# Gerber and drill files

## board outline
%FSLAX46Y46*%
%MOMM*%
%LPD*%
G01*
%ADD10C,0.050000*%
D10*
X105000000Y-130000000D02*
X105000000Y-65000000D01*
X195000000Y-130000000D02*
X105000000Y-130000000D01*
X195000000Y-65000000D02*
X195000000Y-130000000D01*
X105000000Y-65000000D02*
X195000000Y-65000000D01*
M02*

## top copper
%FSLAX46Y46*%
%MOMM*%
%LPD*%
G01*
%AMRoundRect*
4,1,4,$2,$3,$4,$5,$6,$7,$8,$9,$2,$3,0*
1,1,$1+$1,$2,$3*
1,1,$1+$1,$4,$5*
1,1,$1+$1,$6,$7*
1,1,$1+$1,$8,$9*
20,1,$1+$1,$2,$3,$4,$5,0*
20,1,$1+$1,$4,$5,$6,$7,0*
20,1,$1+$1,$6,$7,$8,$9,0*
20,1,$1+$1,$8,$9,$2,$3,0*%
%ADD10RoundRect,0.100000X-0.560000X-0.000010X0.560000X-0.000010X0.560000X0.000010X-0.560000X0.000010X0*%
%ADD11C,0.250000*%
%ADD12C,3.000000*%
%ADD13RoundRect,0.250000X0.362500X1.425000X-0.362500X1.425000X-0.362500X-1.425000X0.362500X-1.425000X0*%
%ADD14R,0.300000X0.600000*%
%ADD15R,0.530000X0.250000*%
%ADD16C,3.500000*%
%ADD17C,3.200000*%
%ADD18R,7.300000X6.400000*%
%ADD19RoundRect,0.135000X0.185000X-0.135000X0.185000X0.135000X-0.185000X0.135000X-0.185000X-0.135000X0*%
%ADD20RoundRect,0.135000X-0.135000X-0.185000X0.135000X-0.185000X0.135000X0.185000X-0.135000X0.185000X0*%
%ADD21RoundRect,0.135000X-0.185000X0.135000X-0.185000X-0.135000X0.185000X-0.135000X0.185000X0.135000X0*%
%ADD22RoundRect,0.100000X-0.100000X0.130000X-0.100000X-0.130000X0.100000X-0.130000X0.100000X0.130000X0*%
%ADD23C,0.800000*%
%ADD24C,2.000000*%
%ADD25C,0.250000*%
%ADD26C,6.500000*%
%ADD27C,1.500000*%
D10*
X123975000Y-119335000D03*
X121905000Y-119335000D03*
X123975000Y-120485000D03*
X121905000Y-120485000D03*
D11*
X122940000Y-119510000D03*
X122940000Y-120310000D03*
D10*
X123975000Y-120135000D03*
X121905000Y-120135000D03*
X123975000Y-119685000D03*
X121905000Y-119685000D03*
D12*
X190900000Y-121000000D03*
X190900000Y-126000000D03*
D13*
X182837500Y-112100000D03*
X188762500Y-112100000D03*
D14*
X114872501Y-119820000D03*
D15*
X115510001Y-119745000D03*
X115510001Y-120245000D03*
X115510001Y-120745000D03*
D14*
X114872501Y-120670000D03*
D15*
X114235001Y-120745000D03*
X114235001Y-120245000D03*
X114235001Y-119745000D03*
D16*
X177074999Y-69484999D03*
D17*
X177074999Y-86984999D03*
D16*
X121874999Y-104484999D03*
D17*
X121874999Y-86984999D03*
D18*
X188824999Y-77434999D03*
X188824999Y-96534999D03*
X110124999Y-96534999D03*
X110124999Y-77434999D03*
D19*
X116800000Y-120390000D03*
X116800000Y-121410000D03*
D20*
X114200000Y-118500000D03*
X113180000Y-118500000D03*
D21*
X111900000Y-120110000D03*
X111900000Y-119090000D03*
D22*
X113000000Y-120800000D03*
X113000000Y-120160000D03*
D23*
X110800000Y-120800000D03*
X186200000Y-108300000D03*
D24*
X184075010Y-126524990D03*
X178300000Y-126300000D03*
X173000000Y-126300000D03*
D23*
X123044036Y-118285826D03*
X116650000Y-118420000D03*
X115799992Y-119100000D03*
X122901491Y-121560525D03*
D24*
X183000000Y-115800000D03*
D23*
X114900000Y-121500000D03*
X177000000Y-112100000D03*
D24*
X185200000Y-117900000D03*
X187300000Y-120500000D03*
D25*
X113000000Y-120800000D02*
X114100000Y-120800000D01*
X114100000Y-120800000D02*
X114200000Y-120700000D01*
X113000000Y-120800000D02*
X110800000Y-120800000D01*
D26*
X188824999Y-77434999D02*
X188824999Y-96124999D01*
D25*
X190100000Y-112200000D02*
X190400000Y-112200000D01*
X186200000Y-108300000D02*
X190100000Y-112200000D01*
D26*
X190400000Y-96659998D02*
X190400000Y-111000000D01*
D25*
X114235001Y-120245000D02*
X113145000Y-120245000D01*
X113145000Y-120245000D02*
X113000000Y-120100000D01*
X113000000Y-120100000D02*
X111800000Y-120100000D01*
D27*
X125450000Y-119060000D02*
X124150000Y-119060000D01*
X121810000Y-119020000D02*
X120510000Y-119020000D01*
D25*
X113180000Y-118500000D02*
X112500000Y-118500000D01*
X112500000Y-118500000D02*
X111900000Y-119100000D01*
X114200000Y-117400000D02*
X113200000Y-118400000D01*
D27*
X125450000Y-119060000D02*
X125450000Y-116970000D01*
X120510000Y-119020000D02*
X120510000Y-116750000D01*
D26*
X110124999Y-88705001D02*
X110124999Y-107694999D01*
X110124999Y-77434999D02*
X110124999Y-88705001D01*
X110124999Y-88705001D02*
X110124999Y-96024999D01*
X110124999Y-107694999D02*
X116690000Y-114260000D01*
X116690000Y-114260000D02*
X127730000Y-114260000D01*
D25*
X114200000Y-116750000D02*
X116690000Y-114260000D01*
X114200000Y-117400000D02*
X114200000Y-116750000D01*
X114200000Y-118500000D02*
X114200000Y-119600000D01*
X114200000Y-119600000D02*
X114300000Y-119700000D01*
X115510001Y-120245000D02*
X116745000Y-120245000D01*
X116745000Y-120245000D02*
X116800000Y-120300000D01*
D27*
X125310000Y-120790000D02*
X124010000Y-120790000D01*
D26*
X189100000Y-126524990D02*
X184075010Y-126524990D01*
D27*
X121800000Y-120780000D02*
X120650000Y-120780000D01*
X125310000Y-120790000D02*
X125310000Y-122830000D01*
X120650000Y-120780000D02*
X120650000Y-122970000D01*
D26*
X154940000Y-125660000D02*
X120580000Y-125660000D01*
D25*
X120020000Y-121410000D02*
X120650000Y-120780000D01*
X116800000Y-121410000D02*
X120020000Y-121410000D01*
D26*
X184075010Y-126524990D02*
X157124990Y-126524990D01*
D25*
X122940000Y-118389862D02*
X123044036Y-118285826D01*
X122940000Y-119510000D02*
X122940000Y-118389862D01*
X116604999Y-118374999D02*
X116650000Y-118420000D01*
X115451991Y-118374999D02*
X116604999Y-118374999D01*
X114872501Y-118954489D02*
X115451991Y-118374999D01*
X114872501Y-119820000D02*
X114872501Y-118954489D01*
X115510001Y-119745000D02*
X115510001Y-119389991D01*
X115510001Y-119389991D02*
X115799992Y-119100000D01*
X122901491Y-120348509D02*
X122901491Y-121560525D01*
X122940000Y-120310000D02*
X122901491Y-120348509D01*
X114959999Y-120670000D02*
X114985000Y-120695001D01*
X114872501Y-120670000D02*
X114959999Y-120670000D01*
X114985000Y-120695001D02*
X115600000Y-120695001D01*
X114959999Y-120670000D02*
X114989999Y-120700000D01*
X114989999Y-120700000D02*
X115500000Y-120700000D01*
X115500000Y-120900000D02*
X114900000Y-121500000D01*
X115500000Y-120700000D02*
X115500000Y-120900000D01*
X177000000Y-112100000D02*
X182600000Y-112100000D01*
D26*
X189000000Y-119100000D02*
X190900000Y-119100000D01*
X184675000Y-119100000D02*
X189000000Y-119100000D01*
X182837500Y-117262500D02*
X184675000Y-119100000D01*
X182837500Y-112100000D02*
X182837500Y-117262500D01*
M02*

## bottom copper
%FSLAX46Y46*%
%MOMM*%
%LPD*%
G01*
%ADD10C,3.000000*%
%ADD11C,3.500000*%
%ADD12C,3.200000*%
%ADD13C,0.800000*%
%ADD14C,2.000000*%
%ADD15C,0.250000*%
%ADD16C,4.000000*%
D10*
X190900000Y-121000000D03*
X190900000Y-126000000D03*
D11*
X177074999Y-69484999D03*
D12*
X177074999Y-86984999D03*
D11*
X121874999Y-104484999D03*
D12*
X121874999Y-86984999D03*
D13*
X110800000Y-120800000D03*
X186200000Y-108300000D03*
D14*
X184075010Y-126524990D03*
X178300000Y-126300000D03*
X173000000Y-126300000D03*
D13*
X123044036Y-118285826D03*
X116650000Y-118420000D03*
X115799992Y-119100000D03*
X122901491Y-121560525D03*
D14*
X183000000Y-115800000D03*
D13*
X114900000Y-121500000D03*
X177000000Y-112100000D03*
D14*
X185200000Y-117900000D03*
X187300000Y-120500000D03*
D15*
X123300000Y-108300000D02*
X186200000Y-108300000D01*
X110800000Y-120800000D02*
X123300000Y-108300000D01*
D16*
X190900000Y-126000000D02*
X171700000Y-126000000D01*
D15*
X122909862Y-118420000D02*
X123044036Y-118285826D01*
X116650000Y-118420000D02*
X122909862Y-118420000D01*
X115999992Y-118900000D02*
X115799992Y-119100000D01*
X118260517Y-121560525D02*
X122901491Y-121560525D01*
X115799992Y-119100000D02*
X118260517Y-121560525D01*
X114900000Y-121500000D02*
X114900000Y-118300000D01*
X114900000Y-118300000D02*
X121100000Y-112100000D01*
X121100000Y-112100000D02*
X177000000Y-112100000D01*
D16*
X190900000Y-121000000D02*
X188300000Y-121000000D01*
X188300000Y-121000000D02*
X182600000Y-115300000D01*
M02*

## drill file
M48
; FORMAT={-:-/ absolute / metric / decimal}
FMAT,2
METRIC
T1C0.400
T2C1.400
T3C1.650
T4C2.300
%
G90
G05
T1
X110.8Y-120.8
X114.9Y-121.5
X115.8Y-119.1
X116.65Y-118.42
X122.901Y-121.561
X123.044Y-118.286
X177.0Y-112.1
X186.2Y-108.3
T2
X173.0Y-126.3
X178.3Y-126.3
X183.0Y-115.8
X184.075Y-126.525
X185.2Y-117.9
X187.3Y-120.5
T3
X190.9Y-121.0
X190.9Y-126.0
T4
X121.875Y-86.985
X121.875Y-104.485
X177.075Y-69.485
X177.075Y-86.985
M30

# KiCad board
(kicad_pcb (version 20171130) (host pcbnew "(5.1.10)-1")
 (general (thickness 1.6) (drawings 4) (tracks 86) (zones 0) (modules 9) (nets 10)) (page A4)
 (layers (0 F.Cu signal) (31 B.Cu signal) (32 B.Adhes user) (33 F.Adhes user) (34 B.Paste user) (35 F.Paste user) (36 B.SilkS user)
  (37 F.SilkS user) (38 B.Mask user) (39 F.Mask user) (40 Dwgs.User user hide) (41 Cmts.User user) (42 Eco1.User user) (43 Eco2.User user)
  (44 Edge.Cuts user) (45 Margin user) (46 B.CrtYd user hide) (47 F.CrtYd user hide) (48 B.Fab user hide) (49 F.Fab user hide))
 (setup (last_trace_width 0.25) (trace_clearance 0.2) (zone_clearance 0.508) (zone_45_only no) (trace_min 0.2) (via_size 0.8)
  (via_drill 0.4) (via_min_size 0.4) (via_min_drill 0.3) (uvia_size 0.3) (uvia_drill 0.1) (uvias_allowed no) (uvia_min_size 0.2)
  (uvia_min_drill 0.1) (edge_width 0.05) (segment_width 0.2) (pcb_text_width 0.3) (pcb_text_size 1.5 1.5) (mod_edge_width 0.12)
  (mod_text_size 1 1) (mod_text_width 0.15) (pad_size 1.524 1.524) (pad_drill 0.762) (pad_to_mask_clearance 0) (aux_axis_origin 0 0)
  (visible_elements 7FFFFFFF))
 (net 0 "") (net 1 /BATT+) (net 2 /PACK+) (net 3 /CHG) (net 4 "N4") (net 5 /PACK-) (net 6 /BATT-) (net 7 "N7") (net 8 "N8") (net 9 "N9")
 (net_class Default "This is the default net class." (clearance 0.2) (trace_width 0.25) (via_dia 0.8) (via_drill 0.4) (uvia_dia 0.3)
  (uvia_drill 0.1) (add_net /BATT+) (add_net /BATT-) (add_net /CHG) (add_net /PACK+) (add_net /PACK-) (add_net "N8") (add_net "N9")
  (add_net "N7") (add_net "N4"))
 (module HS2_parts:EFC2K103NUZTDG (layer F.Cu) (at 122.94 119.91)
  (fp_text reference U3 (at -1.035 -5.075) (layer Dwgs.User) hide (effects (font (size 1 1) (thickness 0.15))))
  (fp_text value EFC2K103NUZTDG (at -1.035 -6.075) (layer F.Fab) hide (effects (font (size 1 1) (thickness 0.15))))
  (pad 1 smd roundrect (at 1.035 -0.575) (size 1.32 0.2) (layers F.Cu F.Paste F.Mask) (roundrect_rratio 0.5) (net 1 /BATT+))
  (pad 1 smd roundrect (at -1.035 -0.575) (size 1.32 0.2) (layers F.Cu F.Paste F.Mask) (roundrect_rratio 0.5) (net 1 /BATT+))
  (pad 2 smd roundrect (at 1.035 0.575) (size 1.32 0.2) (layers F.Cu F.Paste F.Mask) (roundrect_rratio 0.5) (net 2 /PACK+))
  (pad 2 smd roundrect (at -1.035 0.575) (size 1.32 0.2) (layers F.Cu F.Paste F.Mask) (roundrect_rratio 0.5) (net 2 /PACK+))
  (pad 3 smd circle (at 0 -0.4) (size 0.25 0.25) (layers F.Cu F.Paste F.Mask) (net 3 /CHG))
  (pad 4 smd circle (at 0 0.4) (size 0.25 0.25) (layers F.Cu F.Paste F.Mask) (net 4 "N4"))
  (pad 2 smd roundrect (at 1.035 0.225) (size 1.32 0.2) (layers F.Cu F.Paste F.Mask) (roundrect_rratio 0.5) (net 2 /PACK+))
  (pad 2 smd roundrect (at -1.035 0.225) (size 1.32 0.2) (layers F.Cu F.Paste F.Mask) (roundrect_rratio 0.5) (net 2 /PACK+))
  (pad 1 smd roundrect (at 1.035 -0.225) (size 1.32 0.2) (layers F.Cu F.Paste F.Mask) (roundrect_rratio 0.5) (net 1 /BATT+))
  (pad 1 smd roundrect (at -1.035 -0.225) (size 1.32 0.2) (layers F.Cu F.Paste F.Mask) (roundrect_rratio 0.5) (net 1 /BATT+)))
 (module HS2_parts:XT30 (layer F.Cu) (at 190.9 126 180)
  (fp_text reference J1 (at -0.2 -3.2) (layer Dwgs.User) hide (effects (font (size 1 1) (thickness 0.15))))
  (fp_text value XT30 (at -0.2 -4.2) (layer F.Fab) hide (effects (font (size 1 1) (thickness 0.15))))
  (pad 2 thru_hole circle (at 0 5 180) (size 3 3) (drill 1.65) (layers *.Cu *.Mask) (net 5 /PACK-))
  (pad 1 thru_hole circle (at 0 0 180) (size 3 3) (drill 1.65) (layers *.Cu *.Mask) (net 2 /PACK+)))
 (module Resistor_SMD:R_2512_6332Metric (layer F.Cu) (at 185.8 112.1 180)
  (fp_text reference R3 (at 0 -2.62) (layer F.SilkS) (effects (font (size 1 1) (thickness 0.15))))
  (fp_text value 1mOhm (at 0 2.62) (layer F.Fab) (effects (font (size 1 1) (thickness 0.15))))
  (pad 2 smd roundrect (at 2.9625 0 180) (size 1.225 3.35) (layers F.Cu F.Paste F.Mask) (roundrect_rratio 0.2040816326530612) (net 5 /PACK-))
  (pad 1 smd roundrect (at -2.9625 0 180) (size 1.225 3.35) (layers F.Cu F.Paste F.Mask) (roundrect_rratio 0.2040816326530612)
   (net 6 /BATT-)))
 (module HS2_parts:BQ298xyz (layer F.Cu) (at 114.872501 120.245 270)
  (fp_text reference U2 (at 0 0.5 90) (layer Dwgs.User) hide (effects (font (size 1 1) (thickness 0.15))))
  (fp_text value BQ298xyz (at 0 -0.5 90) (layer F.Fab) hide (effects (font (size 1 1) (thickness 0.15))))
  (pad 8 smd rect (at -0.425 0) (size 0.3 0.6) (layers F.Cu F.Paste F.Mask) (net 3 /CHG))
  (pad 7 smd rect (at -0.5 -0.6375 270) (size 0.25 0.53) (layers F.Cu F.Paste F.Mask) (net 4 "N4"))
  (pad 6 smd rect (at 0 -0.6375 270) (size 0.25 0.53) (layers F.Cu F.Paste F.Mask) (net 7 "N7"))
  (pad 5 smd rect (at 0.5 -0.6375 270) (size 0.25 0.53) (layers F.Cu F.Paste F.Mask) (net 5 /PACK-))
  (pad 4 smd rect (at 0.425 0) (size 0.3 0.6) (layers F.Cu F.Paste F.Mask) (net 5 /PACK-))
  (pad 3 smd rect (at 0.5 0.6375 270) (size 0.25 0.53) (layers F.Cu F.Paste F.Mask) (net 6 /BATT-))
  (pad 2 smd rect (at 0 0.6375 270) (size 0.25 0.53) (layers F.Cu F.Paste F.Mask) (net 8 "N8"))
  (pad 1 smd rect (at -0.5 0.6375 270) (size 0.25 0.53) (layers F.Cu F.Paste F.Mask) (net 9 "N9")))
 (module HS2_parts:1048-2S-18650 (layer F.Cu) (at 121.874999 86.984999)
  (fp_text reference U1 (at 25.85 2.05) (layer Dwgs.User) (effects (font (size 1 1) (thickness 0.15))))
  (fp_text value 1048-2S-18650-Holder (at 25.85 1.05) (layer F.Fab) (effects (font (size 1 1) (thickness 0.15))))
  (pad "" np_thru_hole circle (at 55.2 -17.5) (size 3.5 3.5) (drill 2.3) (layers *.Cu *.Mask))
  (pad "" np_thru_hole circle (at 55.2 0) (size 3.2 3.2) (drill 2.3) (layers *.Cu *.Mask))
  (pad "" np_thru_hole circle (at 0 17.5) (size 3.5 3.5) (drill 2.3) (layers *.Cu *.Mask))
  (pad "" np_thru_hole circle (at 0 0) (size 3.2 3.2) (drill 2.3) (layers *.Cu *.Mask))
  (pad 4 smd rect (at 66.95 -9.55) (size 7.3 6.4) (layers F.Cu F.Paste F.Mask) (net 6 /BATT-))
  (pad 3 smd rect (at 66.95 9.55) (size 7.3 6.4) (layers F.Cu F.Paste F.Mask) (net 6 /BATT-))
  (pad 2 smd rect (at -11.75 9.55) (size 7.3 6.4) (layers F.Cu F.Paste F.Mask) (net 1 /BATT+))
  (pad 1 smd rect (at -11.75 -9.55) (size 7.3 6.4) (layers F.Cu F.Paste F.Mask) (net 1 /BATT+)))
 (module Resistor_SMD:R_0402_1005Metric (layer F.Cu) (at 116.8 120.9 90)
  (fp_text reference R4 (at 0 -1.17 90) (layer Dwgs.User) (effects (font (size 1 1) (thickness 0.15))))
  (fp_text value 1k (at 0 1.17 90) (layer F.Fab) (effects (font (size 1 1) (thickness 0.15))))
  (pad 2 smd roundrect (at 0.51 0 90) (size 0.54 0.64) (layers F.Cu F.Paste F.Mask) (roundrect_rratio 0.25) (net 7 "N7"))
  (pad 1 smd roundrect (at -0.51 0 90) (size 0.54 0.64) (layers F.Cu F.Paste F.Mask) (roundrect_rratio 0.25) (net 2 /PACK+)))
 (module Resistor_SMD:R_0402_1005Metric (layer F.Cu) (at 113.69 118.5)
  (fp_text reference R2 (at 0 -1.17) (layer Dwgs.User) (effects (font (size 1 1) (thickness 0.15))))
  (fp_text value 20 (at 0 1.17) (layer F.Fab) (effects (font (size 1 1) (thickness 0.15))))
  (pad 2 smd roundrect (at 0.51 0) (size 0.54 0.64) (layers F.Cu F.Paste F.Mask) (roundrect_rratio 0.25) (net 9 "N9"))
  (pad 1 smd roundrect (at -0.51 0) (size 0.54 0.64) (layers F.Cu F.Paste F.Mask) (roundrect_rratio 0.25) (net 1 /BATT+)))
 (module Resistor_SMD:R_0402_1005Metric (layer F.Cu) (at 111.9 119.6 270)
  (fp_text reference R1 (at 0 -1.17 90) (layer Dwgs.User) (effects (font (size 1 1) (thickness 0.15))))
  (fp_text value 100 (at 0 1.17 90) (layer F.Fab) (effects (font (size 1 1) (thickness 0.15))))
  (pad 2 smd roundrect (at 0.51 0 270) (size 0.54 0.64) (layers F.Cu F.Paste F.Mask) (roundrect_rratio 0.25) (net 8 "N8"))
  (pad 1 smd roundrect (at -0.51 0 270) (size 0.54 0.64) (layers F.Cu F.Paste F.Mask) (roundrect_rratio 0.25) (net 1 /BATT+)))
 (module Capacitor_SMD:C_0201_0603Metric (layer F.Cu) (at 113 120.48 270)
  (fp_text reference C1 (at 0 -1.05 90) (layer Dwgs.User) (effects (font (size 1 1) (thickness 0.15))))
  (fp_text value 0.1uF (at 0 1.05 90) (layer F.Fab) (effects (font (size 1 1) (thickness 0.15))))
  (pad 2 smd roundrect (at 0.32 0 270) (size 0.46 0.4) (layers F.Cu F.Mask) (roundrect_rratio 0.25) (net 6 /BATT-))
  (pad 1 smd roundrect (at -0.32 0 270) (size 0.46 0.4) (layers F.Cu F.Mask) (roundrect_rratio 0.25) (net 8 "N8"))
  (pad "" smd roundrect (at 0.345 0 270) (size 0.318 0.36) (layers F.Paste) (roundrect_rratio 0.25))
  (pad "" smd roundrect (at -0.345 0 270) (size 0.318 0.36) (layers F.Paste) (roundrect_rratio 0.25)))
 (gr_line (start 105 130) (end 105 65) (layer Edge.Cuts) (width 0.05))
 (gr_line (start 195 130) (end 105 130) (layer Edge.Cuts) (width 0.05))
 (gr_line (start 195 65) (end 195 130) (layer Edge.Cuts) (width 0.05))
 (gr_line (start 105 65) (end 195 65) (layer Edge.Cuts) (width 0.05))
 (segment (start 113 120.8) (end 114.1 120.8) (width 0.25) (layer F.Cu) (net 6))
 (segment (start 114.1 120.8) (end 114.2 120.7) (width 0.25) (layer F.Cu) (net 6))
 (via (at 110.8 120.8) (size 0.8) (drill 0.4) (layers F.Cu B.Cu) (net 6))
 (segment (start 113 120.8) (end 110.8 120.8) (width 0.25) (layer F.Cu) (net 6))
 (segment (start 188.824999 77.434999) (end 188.824999 96.124999) (width 6.5) (layer F.Cu) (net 6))
 (via (at 186.2 108.3) (size 0.8) (drill 0.4) (layers F.Cu B.Cu) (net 6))
 (segment (start 123.3 108.3) (end 186.2 108.3) (width 0.25) (layer B.Cu) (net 6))
 (segment (start 110.8 120.8) (end 123.3 108.3) (width 0.25) (layer B.Cu) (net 6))
 (segment (start 190.1 112.2) (end 190.4 112.2) (width 0.25) (layer F.Cu) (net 6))
 (segment (start 186.2 108.3) (end 190.1 112.2) (width 0.25) (layer F.Cu) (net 6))
 (segment (start 190.4 96.659998) (end 190.4 111) (width 6.5) (layer F.Cu) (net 6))
 (segment (start 114.235001 120.245) (end 113.145 120.245) (width 0.25) (layer F.Cu) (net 8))
 (segment (start 113.145 120.245) (end 113 120.1) (width 0.25) (layer F.Cu) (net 8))
 (segment (start 113 120.1) (end 111.8 120.1) (width 0.25) (layer F.Cu) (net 8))
 (segment (start 125.45 119.06) (end 124.15 119.06) (width 1.5) (layer F.Cu) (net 1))
 (segment (start 121.81 119.02) (end 120.51 119.02) (width 1.5) (layer F.Cu) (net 1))
 (segment (start 113.18 118.5) (end 112.5 118.5) (width 0.25) (layer F.Cu) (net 1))
 (segment (start 112.5 118.5) (end 111.9 119.1) (width 0.25) (layer F.Cu) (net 1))
 (segment (start 114.2 117.4) (end 113.2 118.4) (width 0.25) (layer F.Cu) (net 1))
 (segment (start 125.45 119.06) (end 125.45 116.97) (width 1.5) (layer F.Cu) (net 1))
 (segment (start 120.51 119.02) (end 120.51 116.75) (width 1.5) (layer F.Cu) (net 1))
 (segment (start 110.124999 88.705001) (end 110.124999 107.694999) (width 6.5) (layer F.Cu) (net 1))
 (segment (start 110.124999 77.434999) (end 110.124999 88.705001) (width 6.5) (layer F.Cu) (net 1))
 (segment (start 110.124999 88.705001) (end 110.124999 96.024999) (width 6.5) (layer F.Cu) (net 1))
 (segment (start 110.124999 107.694999) (end 116.69 114.26) (width 6.5) (layer F.Cu) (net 1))
 (segment (start 116.69 114.26) (end 127.73 114.26) (width 6.5) (layer F.Cu) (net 1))
 (segment (start 114.2 116.75) (end 116.69 114.26) (width 0.25) (layer F.Cu) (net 1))
 (segment (start 114.2 117.4) (end 114.2 116.75) (width 0.25) (layer F.Cu) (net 1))
 (segment (start 114.2 118.5) (end 114.2 119.6) (width 0.25) (layer F.Cu) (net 9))
 (segment (start 114.2 119.6) (end 114.3 119.7) (width 0.25) (layer F.Cu) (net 9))
 (segment (start 115.510001 120.245) (end 116.745 120.245) (width 0.25) (layer F.Cu) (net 7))
 (segment (start 116.745 120.245) (end 116.8 120.3) (width 0.25) (layer F.Cu) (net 7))
 (segment (start 125.31 120.79) (end 124.01 120.79) (width 1.5) (layer F.Cu) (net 2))
 (segment (start 190.9 126) (end 171.7 126) (width 4) (layer B.Cu) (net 2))
 (segment (start 189.1 126.52499) (end 184.07501 126.52499) (width 6.5) (layer F.Cu) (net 2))
 (via (at 184.07501 126.52499) (size 2) (drill 1.4) (layers F.Cu B.Cu) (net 2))
 (via (at 178.3 126.3) (size 2) (drill 1.4) (layers F.Cu B.Cu) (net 2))
 (via (at 173 126.3) (size 2) (drill 1.4) (layers F.Cu B.Cu) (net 2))
 (segment (start 121.8 120.78) (end 120.65 120.78) (width 1.5) (layer F.Cu) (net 2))
 (segment (start 125.31 120.79) (end 125.31 122.83) (width 1.5) (layer F.Cu) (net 2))
 (segment (start 120.65 120.78) (end 120.65 122.97) (width 1.5) (layer F.Cu) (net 2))
 (segment (start 154.94 125.66) (end 120.58 125.66) (width 6.5) (layer F.Cu) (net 2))
 (segment (start 120.02 121.41) (end 120.65 120.78) (width 0.25) (layer F.Cu) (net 2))
 (segment (start 116.8 121.41) (end 120.02 121.41) (width 0.25) (layer F.Cu) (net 2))
 (segment (start 184.07501 126.52499) (end 157.12499 126.52499) (width 6.5) (layer F.Cu) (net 2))
 (via (at 123.044036 118.285826) (size 0.8) (drill 0.4) (layers F.Cu B.Cu) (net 3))
 (segment (start 122.94 118.389862) (end 123.044036 118.285826) (width 0.25) (layer F.Cu) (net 3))
 (segment (start 122.94 119.51) (end 122.94 118.389862) (width 0.25) (layer F.Cu) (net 3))
 (segment (start 116.604999 118.374999) (end 116.65 118.42) (width 0.25) (layer F.Cu) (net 3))
 (segment (start 115.451991 118.374999) (end 116.604999 118.374999) (width 0.25) (layer F.Cu) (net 3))
 (via (at 116.65 118.42) (size 0.8) (drill 0.4) (layers F.Cu B.Cu) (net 3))
 (segment (start 114.872501 118.954489) (end 115.451991 118.374999) (width 0.25) (layer F.Cu) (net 3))
 (segment (start 114.872501 119.82) (end 114.872501 118.954489) (width 0.25) (layer F.Cu) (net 3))
 (segment (start 122.909862 118.42) (end 123.044036 118.285826) (width 0.25) (layer B.Cu) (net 3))
 (segment (start 116.65 118.42) (end 122.909862 118.42) (width 0.25) (layer B.Cu) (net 3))
 (via (at 115.799992 119.1) (size 0.8) (drill 0.4) (layers F.Cu B.Cu) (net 4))
 (segment (start 115.510001 119.745) (end 115.510001 119.389991) (width 0.25) (layer F.Cu) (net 4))
 (segment (start 115.510001 119.389991) (end 115.799992 119.1) (width 0.25) (layer F.Cu) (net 4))
 (segment (start 115.999992 118.9) (end 115.799992 119.1) (width 0.25) (layer B.Cu) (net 4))
 (segment (start 122.901491 120.348509) (end 122.901491 121.560525) (width 0.25) (layer F.Cu) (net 4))
 (via (at 122.901491 121.560525) (size 0.8) (drill 0.4) (layers F.Cu B.Cu) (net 4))
 (segment (start 122.94 120.31) (end 122.901491 120.348509) (width 0.25) (layer F.Cu) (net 4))
 (segment (start 118.260517 121.560525) (end 122.901491 121.560525) (width 0.25) (layer B.Cu) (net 4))
 (segment (start 115.799992 119.1) (end 118.260517 121.560525) (width 0.25) (layer B.Cu) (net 4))
 (via (at 183 115.8) (size 2) (drill 1.4) (layers F.Cu B.Cu) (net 5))
 (segment (start 114.959999 120.67) (end 114.985 120.695001) (width 0.25) (layer F.Cu) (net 5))
 (segment (start 114.872501 120.67) (end 114.959999 120.67) (width 0.25) (layer F.Cu) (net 5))
 (segment (start 114.985 120.695001) (end 115.6 120.695001) (width 0.25) (layer F.Cu) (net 5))
 (segment (start 114.959999 120.67) (end 114.989999 120.7) (width 0.25) (layer F.Cu) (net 5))
 (segment (start 114.989999 120.7) (end 115.5 120.7) (width 0.25) (layer F.Cu) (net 5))
 (via (at 114.9 121.5) (size 0.8) (drill 0.4) (layers F.Cu B.Cu) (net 5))
 (segment (start 115.5 120.9) (end 114.9 121.5) (width 0.25) (layer F.Cu) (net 5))
 (segment (start 115.5 120.7) (end 115.5 120.9) (width 0.25) (layer F.Cu) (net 5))
 (via (at 177 112.1) (size 0.8) (drill 0.4) (layers F.Cu B.Cu) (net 5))
 (segment (start 114.9 121.5) (end 114.9 118.3) (width 0.25) (layer B.Cu) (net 5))
 (segment (start 114.9 118.3) (end 121.1 112.1) (width 0.25) (layer B.Cu) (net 5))
 (segment (start 121.1 112.1) (end 177 112.1) (width 0.25) (layer B.Cu) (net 5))
 (segment (start 177 112.1) (end 182.6 112.1) (width 0.25) (layer F.Cu) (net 5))
 (segment (start 190.9 121) (end 188.3 121) (width 4) (layer B.Cu) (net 5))
 (segment (start 188.3 121) (end 182.6 115.3) (width 4) (layer B.Cu) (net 5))
 (via (at 185.2 117.9) (size 2) (drill 1.4) (layers F.Cu B.Cu) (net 5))
 (via (at 187.3 120.5) (size 2) (drill 1.4) (layers F.Cu B.Cu) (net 5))
 (segment (start 189 119.1) (end 190.9 119.1) (width 6.5) (layer F.Cu) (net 5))
 (segment (start 184.675 119.1) (end 189 119.1) (width 6.5) (layer F.Cu) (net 5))
 (segment (start 182.8375 117.2625) (end 184.675 119.1) (width 6.5) (layer F.Cu) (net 5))
 (segment (start 182.8375 112.1) (end 182.8375 117.2625) (width 6.5) (layer F.Cu) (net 5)))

